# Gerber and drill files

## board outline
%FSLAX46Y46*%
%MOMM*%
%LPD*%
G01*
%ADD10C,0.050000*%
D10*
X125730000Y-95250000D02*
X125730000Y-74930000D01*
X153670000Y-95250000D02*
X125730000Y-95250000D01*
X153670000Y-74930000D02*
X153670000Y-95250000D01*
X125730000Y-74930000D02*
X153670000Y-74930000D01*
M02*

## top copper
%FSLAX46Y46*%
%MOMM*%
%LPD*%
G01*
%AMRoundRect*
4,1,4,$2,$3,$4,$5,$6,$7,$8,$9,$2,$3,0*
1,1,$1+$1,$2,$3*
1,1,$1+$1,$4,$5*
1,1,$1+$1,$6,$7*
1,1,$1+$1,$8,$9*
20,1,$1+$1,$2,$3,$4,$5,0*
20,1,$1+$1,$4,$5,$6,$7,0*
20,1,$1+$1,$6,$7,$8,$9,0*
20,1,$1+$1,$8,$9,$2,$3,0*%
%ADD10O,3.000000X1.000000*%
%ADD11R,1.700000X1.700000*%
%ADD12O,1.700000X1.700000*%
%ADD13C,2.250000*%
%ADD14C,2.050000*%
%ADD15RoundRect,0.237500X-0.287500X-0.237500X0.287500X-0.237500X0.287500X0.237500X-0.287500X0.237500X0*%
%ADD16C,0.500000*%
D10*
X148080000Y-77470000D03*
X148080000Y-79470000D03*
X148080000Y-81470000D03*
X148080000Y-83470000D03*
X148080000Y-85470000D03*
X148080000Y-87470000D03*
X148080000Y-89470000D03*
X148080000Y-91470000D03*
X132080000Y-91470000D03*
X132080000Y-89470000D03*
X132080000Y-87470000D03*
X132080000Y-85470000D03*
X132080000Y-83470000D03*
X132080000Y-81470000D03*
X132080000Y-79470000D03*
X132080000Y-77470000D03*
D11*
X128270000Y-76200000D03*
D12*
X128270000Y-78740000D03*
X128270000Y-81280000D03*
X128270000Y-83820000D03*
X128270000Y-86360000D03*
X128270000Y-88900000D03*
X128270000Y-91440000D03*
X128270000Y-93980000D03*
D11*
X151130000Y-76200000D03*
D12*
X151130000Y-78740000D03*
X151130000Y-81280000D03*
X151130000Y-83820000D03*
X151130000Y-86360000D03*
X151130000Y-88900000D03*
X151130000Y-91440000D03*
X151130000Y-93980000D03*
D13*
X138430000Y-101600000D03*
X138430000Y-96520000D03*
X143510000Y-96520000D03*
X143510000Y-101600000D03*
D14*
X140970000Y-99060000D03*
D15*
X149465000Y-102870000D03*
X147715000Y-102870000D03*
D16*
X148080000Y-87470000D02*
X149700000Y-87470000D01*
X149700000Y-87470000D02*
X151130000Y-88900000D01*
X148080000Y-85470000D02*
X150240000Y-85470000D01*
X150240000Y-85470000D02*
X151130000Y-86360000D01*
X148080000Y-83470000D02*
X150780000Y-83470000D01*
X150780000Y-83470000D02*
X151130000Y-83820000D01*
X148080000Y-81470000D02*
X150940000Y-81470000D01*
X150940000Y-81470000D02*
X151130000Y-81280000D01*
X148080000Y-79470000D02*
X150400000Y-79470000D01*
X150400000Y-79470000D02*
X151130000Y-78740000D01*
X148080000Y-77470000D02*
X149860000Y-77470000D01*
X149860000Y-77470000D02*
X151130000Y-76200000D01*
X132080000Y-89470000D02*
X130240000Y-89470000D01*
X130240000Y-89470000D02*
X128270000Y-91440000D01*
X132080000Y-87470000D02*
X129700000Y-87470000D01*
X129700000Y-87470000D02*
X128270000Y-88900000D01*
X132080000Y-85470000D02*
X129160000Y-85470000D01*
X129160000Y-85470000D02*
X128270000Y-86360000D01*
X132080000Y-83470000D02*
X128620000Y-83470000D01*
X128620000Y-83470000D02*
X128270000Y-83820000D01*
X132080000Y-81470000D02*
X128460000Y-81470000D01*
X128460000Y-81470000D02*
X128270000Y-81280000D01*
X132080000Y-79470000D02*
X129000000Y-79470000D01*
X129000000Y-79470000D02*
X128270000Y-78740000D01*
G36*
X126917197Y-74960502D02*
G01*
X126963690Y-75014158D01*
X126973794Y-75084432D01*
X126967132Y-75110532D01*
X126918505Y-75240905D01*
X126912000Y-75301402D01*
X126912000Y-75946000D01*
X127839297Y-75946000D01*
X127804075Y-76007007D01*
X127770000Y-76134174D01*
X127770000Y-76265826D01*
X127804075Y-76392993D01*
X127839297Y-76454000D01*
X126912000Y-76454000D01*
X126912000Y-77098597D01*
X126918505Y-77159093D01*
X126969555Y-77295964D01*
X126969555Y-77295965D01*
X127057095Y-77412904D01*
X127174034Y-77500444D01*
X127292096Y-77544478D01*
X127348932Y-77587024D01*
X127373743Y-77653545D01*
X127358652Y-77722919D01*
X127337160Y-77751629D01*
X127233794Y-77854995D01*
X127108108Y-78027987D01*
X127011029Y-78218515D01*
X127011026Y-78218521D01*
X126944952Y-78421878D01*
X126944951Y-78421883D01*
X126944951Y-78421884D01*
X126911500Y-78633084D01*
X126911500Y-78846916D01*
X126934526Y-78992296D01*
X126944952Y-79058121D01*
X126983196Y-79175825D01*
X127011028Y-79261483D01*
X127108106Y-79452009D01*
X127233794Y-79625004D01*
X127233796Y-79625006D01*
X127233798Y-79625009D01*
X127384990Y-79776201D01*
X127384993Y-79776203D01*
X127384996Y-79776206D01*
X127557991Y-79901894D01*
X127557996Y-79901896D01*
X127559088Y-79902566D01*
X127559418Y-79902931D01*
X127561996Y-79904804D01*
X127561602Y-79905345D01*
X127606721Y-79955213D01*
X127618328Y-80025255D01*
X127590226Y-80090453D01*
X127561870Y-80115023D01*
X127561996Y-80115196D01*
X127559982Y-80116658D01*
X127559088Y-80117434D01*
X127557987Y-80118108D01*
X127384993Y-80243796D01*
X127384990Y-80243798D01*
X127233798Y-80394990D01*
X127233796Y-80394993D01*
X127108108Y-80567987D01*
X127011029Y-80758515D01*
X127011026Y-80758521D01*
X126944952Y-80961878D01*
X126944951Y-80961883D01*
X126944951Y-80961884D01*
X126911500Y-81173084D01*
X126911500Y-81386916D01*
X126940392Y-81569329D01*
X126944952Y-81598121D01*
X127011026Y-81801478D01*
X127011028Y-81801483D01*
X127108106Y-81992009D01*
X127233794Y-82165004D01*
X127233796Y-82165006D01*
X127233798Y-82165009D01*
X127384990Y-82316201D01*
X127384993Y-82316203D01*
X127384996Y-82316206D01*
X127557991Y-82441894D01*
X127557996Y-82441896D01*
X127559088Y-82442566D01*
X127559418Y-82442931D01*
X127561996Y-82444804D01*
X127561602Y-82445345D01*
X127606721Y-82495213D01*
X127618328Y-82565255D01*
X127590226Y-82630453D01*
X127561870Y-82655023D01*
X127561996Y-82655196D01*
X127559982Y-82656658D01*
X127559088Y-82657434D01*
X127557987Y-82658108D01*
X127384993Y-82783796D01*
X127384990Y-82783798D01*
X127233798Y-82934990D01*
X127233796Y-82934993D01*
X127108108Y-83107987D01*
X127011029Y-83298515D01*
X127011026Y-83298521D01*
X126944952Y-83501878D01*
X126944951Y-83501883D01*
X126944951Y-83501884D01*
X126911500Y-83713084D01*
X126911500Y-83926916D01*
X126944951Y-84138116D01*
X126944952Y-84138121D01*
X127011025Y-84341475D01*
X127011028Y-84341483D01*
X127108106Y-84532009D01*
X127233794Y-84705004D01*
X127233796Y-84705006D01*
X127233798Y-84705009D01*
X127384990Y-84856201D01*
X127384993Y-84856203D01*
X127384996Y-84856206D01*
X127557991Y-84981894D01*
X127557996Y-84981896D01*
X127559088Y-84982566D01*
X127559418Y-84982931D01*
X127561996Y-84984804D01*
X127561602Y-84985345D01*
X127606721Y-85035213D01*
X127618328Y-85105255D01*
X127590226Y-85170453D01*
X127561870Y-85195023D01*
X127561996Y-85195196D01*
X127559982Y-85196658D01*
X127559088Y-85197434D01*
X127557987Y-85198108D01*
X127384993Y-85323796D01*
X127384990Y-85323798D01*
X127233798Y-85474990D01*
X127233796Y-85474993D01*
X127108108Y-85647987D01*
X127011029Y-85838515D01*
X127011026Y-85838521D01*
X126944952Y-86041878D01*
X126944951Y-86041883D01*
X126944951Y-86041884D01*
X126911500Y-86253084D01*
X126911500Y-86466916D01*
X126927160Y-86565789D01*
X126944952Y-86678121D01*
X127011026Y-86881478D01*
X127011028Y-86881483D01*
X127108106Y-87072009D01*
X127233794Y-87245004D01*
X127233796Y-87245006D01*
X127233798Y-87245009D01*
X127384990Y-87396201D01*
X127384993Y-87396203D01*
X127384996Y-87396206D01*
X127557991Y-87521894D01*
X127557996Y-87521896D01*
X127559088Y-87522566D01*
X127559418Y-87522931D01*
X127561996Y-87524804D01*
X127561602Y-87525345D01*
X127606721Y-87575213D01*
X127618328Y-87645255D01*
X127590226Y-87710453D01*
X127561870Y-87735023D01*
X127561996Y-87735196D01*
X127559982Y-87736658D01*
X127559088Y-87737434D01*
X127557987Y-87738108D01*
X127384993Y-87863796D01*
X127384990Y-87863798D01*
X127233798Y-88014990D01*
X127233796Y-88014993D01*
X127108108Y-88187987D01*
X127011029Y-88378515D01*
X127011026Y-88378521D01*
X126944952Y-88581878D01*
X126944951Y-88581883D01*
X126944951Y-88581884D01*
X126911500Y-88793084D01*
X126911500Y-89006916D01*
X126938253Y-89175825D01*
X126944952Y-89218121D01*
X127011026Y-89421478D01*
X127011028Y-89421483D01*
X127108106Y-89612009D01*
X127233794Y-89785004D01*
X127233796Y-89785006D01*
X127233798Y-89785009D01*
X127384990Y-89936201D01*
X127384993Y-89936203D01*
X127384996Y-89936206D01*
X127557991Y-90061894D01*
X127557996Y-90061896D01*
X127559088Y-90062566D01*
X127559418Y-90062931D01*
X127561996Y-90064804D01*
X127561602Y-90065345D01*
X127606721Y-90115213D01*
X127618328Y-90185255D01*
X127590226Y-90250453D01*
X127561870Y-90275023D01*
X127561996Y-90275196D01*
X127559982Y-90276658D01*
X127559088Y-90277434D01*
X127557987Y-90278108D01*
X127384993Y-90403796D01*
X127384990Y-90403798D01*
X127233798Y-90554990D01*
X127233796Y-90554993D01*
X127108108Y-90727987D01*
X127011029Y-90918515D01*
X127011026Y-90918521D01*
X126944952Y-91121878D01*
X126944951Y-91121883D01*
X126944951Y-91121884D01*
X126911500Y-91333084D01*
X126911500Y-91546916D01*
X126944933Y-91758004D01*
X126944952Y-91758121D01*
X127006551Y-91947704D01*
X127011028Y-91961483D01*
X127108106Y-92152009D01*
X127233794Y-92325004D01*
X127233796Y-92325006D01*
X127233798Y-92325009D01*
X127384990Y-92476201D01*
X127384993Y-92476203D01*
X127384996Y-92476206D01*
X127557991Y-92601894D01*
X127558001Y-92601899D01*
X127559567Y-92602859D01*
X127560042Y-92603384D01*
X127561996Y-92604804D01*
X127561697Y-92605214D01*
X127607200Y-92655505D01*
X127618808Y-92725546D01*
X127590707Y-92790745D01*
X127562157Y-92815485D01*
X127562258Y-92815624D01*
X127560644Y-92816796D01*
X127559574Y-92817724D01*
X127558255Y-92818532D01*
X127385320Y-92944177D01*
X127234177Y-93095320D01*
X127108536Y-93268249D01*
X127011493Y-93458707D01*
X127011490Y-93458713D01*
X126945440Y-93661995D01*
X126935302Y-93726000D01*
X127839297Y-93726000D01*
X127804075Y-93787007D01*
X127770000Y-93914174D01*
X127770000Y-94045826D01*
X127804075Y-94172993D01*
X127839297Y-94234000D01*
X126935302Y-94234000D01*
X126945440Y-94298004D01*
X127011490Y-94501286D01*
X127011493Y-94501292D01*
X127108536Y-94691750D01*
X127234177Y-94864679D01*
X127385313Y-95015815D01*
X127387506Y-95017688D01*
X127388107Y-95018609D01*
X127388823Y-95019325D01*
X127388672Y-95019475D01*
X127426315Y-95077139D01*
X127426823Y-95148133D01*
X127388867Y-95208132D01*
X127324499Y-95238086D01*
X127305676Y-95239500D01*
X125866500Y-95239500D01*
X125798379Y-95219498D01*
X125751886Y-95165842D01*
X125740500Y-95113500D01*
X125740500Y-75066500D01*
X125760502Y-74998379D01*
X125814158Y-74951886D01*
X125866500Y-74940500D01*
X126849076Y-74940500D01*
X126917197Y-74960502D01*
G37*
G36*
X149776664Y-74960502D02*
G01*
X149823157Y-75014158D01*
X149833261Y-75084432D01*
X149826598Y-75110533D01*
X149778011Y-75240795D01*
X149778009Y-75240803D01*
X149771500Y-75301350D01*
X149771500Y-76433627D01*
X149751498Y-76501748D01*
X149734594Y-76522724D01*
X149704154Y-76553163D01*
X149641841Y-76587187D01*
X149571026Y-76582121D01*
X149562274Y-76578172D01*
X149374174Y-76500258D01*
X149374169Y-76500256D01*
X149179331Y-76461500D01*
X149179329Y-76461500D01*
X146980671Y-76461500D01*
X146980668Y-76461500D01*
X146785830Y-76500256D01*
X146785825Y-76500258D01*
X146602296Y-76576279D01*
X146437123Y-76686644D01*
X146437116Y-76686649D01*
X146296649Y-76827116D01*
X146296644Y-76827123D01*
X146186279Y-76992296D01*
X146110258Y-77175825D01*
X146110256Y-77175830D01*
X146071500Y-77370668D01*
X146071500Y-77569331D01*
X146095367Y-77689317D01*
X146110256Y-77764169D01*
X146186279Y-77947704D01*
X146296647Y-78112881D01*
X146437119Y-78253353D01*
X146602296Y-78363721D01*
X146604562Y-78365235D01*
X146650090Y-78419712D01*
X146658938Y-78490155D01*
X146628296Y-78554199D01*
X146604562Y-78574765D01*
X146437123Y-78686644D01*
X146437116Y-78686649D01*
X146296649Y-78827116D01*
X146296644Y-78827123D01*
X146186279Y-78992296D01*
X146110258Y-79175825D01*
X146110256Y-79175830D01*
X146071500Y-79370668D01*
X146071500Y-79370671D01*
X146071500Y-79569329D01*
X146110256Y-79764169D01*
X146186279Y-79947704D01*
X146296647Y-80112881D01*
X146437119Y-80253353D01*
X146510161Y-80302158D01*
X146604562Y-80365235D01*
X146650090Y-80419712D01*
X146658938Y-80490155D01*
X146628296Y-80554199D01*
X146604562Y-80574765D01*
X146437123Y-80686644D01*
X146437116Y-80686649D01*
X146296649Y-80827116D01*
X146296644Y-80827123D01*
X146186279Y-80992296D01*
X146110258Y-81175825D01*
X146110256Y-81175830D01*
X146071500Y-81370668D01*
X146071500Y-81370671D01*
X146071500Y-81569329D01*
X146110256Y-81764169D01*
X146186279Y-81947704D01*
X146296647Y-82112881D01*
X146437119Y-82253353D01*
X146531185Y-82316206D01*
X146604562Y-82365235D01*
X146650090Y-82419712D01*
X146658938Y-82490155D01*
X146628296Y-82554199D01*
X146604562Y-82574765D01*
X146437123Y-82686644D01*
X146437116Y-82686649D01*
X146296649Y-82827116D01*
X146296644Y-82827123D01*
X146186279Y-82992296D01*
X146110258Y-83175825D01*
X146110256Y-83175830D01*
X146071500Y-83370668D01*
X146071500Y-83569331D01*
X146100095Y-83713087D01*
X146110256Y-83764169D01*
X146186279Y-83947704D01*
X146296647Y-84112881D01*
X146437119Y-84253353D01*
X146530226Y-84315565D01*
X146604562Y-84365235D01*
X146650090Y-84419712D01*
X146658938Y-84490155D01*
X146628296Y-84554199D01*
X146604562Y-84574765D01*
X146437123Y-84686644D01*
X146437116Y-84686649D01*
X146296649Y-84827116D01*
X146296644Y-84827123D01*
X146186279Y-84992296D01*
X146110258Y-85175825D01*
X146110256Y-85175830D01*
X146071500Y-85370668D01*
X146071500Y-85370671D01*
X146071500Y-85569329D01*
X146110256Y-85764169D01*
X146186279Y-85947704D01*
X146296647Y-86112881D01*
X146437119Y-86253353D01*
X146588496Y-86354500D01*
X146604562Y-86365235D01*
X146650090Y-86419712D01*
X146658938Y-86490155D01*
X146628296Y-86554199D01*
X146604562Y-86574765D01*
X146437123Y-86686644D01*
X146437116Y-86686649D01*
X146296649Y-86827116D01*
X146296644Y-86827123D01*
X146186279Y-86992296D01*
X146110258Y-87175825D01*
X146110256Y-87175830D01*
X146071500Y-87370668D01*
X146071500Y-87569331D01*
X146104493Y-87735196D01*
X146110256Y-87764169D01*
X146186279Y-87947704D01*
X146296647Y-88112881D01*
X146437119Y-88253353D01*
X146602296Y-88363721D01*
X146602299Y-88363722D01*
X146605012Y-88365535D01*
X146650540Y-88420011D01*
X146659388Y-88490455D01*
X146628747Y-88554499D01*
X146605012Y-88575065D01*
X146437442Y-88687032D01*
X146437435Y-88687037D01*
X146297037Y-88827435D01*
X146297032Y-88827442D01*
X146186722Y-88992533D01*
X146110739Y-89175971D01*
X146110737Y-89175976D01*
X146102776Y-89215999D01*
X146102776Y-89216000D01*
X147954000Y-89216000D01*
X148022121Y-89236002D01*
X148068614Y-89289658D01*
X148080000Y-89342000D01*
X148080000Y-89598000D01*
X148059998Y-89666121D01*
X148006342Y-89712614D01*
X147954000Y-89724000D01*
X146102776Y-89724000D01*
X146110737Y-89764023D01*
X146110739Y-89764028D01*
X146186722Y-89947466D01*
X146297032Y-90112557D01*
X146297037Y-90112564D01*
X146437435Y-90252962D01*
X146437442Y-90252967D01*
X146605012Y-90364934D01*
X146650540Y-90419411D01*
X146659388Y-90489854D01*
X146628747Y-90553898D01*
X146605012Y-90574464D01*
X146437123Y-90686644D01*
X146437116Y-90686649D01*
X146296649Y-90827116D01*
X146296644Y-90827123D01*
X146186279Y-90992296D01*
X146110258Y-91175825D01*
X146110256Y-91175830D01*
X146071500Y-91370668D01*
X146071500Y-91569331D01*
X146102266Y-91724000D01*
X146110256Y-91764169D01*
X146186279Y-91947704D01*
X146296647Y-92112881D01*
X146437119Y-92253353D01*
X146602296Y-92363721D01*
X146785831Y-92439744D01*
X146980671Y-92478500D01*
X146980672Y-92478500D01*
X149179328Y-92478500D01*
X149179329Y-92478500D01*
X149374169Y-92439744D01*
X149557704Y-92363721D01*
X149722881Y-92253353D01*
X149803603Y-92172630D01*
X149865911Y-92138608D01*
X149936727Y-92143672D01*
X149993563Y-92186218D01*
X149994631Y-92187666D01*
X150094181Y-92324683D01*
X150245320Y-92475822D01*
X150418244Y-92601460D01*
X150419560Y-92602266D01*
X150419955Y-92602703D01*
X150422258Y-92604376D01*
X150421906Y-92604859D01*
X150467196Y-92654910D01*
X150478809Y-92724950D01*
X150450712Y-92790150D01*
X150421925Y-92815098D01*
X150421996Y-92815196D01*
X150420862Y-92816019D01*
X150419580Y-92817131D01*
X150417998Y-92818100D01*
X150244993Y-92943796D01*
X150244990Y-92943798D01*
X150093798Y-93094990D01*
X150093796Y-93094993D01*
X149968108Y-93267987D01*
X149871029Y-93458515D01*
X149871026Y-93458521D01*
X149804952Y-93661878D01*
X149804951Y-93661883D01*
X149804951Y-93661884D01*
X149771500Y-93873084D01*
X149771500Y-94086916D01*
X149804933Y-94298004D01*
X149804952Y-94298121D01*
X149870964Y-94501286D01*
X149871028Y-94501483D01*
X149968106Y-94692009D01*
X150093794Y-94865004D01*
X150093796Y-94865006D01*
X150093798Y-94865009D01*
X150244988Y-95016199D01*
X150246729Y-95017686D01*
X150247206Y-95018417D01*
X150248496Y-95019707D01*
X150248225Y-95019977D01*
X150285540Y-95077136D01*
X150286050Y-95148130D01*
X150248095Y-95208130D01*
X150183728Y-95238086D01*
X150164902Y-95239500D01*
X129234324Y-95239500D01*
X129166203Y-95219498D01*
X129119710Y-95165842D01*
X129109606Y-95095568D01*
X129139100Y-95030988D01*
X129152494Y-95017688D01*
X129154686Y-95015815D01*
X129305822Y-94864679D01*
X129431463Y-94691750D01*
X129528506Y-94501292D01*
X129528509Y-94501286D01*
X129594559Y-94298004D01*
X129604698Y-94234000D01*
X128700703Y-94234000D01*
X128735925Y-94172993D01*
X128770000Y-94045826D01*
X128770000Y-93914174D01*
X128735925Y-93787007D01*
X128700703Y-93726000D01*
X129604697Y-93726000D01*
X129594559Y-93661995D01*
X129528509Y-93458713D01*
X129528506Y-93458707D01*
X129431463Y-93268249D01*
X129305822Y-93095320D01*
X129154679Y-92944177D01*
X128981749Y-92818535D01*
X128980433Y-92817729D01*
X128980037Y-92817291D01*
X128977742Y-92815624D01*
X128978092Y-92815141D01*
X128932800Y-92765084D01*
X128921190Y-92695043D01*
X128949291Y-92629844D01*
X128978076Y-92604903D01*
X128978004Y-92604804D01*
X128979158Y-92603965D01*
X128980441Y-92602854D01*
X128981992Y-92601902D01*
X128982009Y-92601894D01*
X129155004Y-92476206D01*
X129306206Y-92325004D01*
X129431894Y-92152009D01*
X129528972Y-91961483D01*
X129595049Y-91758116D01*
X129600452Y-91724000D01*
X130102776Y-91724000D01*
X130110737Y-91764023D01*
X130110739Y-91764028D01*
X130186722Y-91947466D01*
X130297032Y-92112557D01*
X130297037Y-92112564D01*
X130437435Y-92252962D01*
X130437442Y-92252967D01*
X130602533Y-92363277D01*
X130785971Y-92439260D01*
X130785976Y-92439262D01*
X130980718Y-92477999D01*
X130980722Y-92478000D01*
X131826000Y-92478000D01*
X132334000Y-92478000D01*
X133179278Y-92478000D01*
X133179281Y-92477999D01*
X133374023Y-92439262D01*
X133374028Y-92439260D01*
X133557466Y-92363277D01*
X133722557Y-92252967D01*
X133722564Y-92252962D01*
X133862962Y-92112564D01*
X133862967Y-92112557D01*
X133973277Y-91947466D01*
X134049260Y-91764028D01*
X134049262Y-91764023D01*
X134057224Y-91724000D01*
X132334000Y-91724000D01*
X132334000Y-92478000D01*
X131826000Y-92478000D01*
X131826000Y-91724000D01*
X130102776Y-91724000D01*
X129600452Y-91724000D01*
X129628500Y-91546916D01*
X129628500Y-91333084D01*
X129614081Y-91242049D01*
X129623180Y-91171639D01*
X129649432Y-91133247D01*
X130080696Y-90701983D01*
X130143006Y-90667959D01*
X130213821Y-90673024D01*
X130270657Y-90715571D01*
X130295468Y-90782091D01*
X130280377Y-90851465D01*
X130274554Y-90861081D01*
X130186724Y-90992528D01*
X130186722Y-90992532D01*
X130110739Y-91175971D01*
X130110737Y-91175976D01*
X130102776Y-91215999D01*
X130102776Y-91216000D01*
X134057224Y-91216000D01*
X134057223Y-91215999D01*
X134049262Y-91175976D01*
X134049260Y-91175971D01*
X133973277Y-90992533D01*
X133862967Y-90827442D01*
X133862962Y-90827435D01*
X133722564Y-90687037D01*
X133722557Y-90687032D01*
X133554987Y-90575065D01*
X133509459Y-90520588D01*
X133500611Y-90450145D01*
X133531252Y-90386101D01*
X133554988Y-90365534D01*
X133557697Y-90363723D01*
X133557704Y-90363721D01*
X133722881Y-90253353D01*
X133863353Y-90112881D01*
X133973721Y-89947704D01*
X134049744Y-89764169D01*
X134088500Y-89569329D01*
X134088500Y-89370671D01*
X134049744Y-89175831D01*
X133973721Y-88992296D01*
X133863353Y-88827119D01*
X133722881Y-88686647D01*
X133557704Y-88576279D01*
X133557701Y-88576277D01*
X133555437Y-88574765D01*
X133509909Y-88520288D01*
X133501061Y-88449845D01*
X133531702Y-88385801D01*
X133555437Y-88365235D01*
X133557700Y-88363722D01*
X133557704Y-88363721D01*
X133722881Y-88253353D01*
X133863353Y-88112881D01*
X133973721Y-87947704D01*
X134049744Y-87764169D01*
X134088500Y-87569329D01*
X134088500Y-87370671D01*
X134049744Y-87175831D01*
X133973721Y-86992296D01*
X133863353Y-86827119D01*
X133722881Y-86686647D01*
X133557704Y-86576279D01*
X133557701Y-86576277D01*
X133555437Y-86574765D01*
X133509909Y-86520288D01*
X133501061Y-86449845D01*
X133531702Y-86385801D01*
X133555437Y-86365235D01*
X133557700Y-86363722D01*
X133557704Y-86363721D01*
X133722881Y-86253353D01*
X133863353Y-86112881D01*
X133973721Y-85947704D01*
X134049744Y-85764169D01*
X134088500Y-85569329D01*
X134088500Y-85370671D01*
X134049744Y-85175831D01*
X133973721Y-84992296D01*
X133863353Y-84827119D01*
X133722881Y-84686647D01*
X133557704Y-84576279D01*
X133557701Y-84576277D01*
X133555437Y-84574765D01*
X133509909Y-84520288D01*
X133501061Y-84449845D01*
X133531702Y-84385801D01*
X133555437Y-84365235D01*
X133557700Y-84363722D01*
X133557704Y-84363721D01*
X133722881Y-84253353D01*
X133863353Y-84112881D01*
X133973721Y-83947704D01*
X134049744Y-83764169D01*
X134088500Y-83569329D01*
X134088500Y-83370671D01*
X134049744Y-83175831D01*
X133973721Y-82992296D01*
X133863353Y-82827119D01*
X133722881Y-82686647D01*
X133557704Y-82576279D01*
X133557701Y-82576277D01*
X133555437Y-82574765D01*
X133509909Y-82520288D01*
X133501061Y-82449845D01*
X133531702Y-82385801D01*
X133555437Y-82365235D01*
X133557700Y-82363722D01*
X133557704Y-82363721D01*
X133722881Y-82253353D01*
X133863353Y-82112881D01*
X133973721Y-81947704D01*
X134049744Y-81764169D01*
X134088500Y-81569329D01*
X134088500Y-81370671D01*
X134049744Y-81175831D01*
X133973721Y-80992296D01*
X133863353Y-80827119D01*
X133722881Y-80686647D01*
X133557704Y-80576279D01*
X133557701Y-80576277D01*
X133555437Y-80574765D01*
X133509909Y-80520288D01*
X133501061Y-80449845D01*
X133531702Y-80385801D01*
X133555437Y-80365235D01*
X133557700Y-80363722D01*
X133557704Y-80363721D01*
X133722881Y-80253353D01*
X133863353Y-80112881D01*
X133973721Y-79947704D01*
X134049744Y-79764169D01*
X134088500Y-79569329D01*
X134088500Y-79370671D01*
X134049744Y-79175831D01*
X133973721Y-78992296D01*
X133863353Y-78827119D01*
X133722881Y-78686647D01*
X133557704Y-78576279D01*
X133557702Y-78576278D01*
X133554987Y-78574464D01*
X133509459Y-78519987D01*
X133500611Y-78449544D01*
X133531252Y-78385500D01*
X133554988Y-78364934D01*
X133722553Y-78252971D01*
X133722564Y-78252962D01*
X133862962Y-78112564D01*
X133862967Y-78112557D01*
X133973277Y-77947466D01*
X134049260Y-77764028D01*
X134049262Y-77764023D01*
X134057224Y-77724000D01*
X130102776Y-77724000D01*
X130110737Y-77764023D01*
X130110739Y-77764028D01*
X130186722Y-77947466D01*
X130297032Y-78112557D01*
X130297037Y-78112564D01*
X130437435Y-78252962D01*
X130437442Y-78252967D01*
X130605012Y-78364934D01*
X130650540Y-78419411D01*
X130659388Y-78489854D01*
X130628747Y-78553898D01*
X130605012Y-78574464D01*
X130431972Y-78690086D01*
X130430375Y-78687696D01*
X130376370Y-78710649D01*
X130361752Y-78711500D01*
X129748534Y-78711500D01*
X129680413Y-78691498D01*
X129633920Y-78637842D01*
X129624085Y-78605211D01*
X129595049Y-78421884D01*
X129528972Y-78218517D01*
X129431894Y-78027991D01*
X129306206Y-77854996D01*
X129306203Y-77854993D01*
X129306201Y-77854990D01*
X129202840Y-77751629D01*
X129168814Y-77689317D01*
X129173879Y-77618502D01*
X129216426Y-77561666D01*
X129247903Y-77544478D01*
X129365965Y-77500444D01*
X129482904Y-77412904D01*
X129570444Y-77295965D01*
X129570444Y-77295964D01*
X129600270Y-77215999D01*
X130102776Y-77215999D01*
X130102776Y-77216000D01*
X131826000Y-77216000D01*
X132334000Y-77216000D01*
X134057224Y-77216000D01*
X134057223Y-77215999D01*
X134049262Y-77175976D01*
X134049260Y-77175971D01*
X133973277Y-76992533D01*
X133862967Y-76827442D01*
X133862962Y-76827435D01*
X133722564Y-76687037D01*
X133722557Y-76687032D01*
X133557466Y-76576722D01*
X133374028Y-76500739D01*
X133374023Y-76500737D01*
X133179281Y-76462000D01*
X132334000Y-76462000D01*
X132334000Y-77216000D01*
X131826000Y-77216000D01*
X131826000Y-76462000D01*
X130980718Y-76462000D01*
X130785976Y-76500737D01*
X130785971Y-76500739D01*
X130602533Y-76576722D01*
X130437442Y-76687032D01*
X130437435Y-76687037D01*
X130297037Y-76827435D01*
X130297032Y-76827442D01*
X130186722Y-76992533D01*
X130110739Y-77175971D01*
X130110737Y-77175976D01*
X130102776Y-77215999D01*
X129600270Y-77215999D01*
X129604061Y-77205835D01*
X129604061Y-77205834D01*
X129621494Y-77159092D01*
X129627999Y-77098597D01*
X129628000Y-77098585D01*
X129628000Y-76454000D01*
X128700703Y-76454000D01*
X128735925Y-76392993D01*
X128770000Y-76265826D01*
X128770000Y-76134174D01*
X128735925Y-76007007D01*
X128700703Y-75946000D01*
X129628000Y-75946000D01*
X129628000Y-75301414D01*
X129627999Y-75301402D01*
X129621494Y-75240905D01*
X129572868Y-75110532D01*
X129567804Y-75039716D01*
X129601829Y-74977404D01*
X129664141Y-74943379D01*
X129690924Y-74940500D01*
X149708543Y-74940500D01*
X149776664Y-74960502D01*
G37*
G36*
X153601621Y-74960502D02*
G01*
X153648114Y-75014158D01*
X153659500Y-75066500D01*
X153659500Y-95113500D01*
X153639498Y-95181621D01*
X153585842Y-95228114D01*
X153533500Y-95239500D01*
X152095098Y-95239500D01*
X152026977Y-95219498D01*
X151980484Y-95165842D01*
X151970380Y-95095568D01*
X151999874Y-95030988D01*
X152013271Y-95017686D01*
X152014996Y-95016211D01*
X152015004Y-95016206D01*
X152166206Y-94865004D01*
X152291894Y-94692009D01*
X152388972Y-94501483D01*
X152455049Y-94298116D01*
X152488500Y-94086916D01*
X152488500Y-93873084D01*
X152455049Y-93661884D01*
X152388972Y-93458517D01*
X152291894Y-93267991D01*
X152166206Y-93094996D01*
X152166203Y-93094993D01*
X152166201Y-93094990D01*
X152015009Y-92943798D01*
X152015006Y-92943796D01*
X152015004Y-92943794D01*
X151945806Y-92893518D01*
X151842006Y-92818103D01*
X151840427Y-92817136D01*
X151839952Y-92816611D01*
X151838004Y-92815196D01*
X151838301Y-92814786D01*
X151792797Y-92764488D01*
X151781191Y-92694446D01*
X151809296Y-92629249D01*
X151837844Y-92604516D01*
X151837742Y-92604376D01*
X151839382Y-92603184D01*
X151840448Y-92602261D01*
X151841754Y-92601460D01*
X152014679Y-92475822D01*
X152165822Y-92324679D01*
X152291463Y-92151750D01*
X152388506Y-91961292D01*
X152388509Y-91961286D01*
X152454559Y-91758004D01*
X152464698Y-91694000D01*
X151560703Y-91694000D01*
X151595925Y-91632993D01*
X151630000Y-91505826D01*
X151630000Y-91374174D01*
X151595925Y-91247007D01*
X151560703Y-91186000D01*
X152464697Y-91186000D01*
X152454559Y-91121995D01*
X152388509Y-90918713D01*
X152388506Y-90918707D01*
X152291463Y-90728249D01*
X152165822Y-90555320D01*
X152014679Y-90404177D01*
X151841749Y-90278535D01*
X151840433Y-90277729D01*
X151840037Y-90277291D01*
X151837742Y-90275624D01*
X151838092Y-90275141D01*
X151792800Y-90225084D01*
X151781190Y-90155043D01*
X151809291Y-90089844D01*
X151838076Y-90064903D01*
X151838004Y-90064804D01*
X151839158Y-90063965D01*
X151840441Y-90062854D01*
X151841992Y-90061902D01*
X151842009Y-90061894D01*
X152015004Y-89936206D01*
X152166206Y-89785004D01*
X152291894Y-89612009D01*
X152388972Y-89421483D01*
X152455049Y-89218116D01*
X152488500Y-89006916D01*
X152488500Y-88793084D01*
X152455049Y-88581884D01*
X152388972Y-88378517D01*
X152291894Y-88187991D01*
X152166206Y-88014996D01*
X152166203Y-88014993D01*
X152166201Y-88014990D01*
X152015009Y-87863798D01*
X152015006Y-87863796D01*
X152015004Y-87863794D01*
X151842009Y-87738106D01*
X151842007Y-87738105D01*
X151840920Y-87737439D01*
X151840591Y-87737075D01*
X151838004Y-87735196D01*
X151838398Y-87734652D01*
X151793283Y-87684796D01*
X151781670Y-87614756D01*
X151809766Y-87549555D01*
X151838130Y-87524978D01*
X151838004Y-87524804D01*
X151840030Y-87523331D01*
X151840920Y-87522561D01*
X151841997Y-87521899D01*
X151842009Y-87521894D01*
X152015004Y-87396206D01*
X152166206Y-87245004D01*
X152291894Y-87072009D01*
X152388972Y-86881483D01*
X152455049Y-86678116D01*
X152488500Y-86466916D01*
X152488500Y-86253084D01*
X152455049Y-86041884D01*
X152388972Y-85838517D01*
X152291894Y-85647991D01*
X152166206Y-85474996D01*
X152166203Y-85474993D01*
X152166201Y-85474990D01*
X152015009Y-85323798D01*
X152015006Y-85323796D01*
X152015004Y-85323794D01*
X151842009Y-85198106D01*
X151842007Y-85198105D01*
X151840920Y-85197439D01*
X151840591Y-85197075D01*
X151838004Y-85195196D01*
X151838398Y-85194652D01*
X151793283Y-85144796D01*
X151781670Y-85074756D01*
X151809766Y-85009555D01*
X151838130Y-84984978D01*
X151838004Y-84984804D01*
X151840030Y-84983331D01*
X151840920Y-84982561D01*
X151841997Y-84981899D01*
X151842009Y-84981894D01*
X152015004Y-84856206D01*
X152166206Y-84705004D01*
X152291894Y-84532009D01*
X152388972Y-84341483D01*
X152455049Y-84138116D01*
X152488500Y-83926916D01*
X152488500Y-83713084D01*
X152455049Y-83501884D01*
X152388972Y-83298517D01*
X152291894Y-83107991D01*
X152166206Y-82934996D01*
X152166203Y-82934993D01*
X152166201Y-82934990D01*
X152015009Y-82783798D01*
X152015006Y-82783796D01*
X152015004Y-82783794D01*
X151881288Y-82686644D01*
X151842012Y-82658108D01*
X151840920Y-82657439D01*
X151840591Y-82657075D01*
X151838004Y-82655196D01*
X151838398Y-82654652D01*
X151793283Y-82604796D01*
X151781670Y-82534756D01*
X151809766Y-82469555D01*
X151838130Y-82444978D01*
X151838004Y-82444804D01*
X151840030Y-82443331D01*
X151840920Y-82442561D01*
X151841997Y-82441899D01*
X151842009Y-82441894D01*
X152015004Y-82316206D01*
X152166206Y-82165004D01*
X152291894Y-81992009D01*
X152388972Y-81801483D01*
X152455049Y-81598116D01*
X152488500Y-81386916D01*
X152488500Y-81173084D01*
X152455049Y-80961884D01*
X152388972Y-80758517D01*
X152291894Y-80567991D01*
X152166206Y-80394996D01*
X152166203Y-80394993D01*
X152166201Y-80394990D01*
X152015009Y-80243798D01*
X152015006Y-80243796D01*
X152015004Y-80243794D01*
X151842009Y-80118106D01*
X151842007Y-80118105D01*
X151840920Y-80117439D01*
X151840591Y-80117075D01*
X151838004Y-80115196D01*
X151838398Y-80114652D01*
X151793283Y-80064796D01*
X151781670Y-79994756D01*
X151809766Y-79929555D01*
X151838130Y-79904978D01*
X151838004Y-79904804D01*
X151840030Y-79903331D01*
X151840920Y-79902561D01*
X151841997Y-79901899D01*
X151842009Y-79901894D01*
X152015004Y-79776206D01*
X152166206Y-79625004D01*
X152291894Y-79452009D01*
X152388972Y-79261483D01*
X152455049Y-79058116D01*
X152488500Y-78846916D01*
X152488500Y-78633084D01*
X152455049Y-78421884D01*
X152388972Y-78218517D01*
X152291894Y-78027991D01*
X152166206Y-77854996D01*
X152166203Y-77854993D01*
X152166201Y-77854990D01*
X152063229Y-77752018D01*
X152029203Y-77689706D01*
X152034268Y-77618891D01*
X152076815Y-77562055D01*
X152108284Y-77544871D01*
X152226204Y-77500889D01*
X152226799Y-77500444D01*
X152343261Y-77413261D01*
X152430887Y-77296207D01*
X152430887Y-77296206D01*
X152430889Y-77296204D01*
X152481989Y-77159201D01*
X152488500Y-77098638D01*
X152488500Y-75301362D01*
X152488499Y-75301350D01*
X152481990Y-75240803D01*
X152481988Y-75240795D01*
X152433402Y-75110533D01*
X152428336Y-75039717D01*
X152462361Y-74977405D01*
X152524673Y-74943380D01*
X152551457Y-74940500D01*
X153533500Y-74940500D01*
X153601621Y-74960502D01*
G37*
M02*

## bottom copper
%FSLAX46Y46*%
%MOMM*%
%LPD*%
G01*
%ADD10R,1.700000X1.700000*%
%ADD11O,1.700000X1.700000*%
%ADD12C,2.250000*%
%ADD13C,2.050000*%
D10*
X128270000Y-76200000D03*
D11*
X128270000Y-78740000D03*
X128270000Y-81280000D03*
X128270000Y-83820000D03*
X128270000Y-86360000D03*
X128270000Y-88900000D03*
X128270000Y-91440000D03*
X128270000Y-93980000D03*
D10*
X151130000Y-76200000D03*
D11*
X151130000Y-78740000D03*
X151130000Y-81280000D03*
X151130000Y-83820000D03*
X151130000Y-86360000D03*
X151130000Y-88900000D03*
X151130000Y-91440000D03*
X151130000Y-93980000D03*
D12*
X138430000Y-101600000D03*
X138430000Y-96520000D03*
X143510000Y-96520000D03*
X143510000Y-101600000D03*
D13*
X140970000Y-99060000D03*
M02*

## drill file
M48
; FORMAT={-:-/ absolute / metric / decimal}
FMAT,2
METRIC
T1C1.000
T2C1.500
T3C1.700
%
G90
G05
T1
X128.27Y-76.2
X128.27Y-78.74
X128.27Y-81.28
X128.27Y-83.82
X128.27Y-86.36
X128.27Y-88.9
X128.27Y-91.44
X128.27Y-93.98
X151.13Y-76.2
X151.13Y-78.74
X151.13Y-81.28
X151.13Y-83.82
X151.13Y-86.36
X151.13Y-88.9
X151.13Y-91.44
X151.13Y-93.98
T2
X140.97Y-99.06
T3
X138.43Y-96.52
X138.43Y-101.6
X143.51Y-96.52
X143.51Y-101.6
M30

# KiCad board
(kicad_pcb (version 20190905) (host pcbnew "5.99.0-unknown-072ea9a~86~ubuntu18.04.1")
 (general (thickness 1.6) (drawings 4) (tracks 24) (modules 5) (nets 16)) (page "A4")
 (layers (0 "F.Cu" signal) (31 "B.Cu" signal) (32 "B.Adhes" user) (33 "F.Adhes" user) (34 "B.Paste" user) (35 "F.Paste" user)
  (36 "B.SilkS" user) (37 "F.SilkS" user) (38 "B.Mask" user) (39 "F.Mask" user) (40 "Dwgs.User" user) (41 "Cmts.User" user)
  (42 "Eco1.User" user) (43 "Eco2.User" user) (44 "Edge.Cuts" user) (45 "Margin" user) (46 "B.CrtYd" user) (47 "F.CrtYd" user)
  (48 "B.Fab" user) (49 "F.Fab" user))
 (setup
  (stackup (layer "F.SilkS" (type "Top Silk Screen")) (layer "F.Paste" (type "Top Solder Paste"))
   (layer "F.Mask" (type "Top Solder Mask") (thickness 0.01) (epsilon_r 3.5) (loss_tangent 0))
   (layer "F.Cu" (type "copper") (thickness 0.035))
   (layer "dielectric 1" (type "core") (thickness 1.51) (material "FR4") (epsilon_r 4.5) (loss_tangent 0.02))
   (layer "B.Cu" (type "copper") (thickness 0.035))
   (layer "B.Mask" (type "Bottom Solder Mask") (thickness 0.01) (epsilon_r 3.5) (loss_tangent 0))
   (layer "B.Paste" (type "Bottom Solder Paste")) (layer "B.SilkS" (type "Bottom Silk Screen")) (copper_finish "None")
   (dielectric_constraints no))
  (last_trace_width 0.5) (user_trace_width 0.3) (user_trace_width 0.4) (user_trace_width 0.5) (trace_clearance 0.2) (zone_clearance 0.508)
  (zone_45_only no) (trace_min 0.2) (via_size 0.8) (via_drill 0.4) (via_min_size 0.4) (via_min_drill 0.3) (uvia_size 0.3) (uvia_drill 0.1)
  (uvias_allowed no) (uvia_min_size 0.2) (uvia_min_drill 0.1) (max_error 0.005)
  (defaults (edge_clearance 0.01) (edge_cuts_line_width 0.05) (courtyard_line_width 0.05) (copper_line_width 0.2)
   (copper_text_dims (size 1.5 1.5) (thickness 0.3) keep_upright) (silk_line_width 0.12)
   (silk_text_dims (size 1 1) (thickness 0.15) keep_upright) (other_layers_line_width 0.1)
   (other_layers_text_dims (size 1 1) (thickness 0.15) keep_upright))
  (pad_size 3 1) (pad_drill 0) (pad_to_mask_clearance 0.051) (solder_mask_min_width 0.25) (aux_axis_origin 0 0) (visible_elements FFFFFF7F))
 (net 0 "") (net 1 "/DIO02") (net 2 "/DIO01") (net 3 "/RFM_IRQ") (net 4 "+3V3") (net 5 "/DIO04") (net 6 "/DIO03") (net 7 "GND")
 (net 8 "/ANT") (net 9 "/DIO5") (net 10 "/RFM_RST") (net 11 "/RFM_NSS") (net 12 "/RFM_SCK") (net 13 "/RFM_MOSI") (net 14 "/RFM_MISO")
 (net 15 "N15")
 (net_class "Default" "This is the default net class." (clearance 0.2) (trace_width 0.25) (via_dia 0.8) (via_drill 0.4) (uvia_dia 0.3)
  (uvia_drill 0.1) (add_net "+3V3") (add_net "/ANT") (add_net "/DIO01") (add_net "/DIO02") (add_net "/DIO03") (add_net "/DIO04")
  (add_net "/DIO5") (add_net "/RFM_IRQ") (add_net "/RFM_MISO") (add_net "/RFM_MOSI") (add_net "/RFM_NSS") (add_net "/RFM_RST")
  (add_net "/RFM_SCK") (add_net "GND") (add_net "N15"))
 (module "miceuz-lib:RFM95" (layer "F.Cu") (at 132.08 77.47)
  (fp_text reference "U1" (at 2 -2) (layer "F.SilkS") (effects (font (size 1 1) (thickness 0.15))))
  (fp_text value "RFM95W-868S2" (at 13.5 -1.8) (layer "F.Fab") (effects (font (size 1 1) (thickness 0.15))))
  (pad "16" smd oval (at 16 0) (size 3 1) (layers "F.Cu" "F.Paste" "F.Mask") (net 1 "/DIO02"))
  (pad "15" smd oval (at 16 2) (size 3 1) (layers "F.Cu" "F.Paste" "F.Mask") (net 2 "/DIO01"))
  (pad "14" smd oval (at 16 4) (size 3 1) (layers "F.Cu" "F.Paste" "F.Mask") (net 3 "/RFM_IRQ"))
  (pad "13" smd oval (at 16 6) (size 3 1) (layers "F.Cu" "F.Paste" "F.Mask") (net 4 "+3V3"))
  (pad "12" smd oval (at 16 8) (size 3 1) (layers "F.Cu" "F.Paste" "F.Mask") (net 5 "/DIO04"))
  (pad "11" smd oval (at 16 10) (size 3 1) (layers "F.Cu" "F.Paste" "F.Mask") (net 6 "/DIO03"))
  (pad "10" smd oval (at 16 12) (size 3 1) (layers "F.Cu" "F.Paste" "F.Mask") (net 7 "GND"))
  (pad "9" smd oval (at 16 14) (size 3 1) (layers "F.Cu" "F.Paste" "F.Mask") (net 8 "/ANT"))
  (pad "8" smd oval (at 0 14) (size 3 1) (layers "F.Cu" "F.Paste" "F.Mask") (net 7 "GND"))
  (pad "7" smd oval (at 0 12) (size 3 1) (layers "F.Cu" "F.Paste" "F.Mask") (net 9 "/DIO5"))
  (pad "6" smd oval (at 0 10) (size 3 1) (layers "F.Cu" "F.Paste" "F.Mask") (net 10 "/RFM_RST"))
  (pad "5" smd oval (at 0 8) (size 3 1) (layers "F.Cu" "F.Paste" "F.Mask") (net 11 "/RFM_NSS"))
  (pad "4" smd oval (at 0 6) (size 3 1) (layers "F.Cu" "F.Paste" "F.Mask") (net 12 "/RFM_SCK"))
  (pad "3" smd oval (at 0 4) (size 3 1) (layers "F.Cu" "F.Paste" "F.Mask") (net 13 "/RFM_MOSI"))
  (pad "2" smd oval (at 0 2) (size 3 1) (layers "F.Cu" "F.Paste" "F.Mask") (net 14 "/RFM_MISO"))
  (pad "1" smd oval (at 0 0) (size 3 1) (layers "F.Cu" "F.Paste" "F.Mask") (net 7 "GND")))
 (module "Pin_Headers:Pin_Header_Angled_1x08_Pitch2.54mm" (layer "F.Cu") (at 128.27 76.2)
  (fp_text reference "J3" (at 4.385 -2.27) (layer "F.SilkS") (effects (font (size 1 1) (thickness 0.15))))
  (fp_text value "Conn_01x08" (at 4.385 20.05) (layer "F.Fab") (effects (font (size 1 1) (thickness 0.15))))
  (pad "1" thru_hole rect (at 0 0) (size 1.7 1.7) (drill 1) (layers *.Cu *.Mask) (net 7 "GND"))
  (pad "2" thru_hole oval (at 0 2.54) (size 1.7 1.7) (drill 1) (layers *.Cu *.Mask) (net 14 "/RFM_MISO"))
  (pad "3" thru_hole oval (at 0 5.08) (size 1.7 1.7) (drill 1) (layers *.Cu *.Mask) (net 13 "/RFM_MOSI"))
  (pad "4" thru_hole oval (at 0 7.62) (size 1.7 1.7) (drill 1) (layers *.Cu *.Mask) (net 12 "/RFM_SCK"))
  (pad "5" thru_hole oval (at 0 10.16) (size 1.7 1.7) (drill 1) (layers *.Cu *.Mask) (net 11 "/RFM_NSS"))
  (pad "6" thru_hole oval (at 0 12.7) (size 1.7 1.7) (drill 1) (layers *.Cu *.Mask) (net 10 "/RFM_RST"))
  (pad "7" thru_hole oval (at 0 15.24) (size 1.7 1.7) (drill 1) (layers *.Cu *.Mask) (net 9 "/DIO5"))
  (pad "8" thru_hole oval (at 0 17.78) (size 1.7 1.7) (drill 1) (layers *.Cu *.Mask) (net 7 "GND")))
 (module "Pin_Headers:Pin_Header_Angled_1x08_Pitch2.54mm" (layer "F.Cu") (at 151.13 76.2)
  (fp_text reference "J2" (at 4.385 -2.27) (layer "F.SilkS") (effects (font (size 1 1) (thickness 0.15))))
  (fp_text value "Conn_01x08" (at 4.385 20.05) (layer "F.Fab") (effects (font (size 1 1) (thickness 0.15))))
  (pad "1" thru_hole rect (at 0 0) (size 1.7 1.7) (drill 1) (layers *.Cu *.Mask) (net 1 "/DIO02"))
  (pad "2" thru_hole oval (at 0 2.54) (size 1.7 1.7) (drill 1) (layers *.Cu *.Mask) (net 2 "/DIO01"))
  (pad "3" thru_hole oval (at 0 5.08) (size 1.7 1.7) (drill 1) (layers *.Cu *.Mask) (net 3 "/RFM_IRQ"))
  (pad "4" thru_hole oval (at 0 7.62) (size 1.7 1.7) (drill 1) (layers *.Cu *.Mask) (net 4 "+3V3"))
  (pad "5" thru_hole oval (at 0 10.16) (size 1.7 1.7) (drill 1) (layers *.Cu *.Mask) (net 5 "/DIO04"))
  (pad "6" thru_hole oval (at 0 12.7) (size 1.7 1.7) (drill 1) (layers *.Cu *.Mask) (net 6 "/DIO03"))
  (pad "7" thru_hole oval (at 0 15.24) (size 1.7 1.7) (drill 1) (layers *.Cu *.Mask) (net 7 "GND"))
  (pad "8" thru_hole oval (at 0 17.78) (size 1.7 1.7) (drill 1) (layers *.Cu *.Mask) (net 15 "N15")))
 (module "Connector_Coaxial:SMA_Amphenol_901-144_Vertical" (layer "F.Cu") (at 140.97 99.06)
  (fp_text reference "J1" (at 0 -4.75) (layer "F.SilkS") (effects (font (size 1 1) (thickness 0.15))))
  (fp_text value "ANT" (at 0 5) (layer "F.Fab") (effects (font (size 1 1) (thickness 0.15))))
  (pad "2" thru_hole circle (at -2.54 2.54) (size 2.25 2.25) (drill 1.7) (layers *.Cu *.Mask) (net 7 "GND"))
  (pad "2" thru_hole circle (at -2.54 -2.54) (size 2.25 2.25) (drill 1.7) (layers *.Cu *.Mask) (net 7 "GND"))
  (pad "2" thru_hole circle (at 2.54 -2.54) (size 2.25 2.25) (drill 1.7) (layers *.Cu *.Mask) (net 7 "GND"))
  (pad "2" thru_hole circle (at 2.54 2.54) (size 2.25 2.25) (drill 1.7) (layers *.Cu *.Mask) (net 7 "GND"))
  (pad "1" thru_hole circle (at 0 0) (size 2.05 2.05) (drill 1.5) (layers *.Cu *.Mask) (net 8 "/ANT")))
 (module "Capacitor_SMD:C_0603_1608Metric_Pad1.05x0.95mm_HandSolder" (layer "F.Cu") (at 148.59 102.87)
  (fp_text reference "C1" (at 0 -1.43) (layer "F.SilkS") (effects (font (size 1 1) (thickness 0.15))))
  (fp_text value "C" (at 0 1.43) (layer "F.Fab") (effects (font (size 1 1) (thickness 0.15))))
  (pad "2" smd roundrect (at 0.875 0) (size 1.05 0.95) (layers "F.Cu" "F.Paste" "F.Mask") (roundrect_rratio 0.25) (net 7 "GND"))
  (pad "1" smd roundrect (at -0.875 0) (size 1.05 0.95) (layers "F.Cu" "F.Paste" "F.Mask") (roundrect_rratio 0.25) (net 4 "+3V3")))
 (gr_line (start 125.73 95.25) (end 125.73 74.93) (layer "Edge.Cuts") (width 0.05))
 (gr_line (start 153.67 95.25) (end 125.73 95.25) (layer "Edge.Cuts") (width 0.05))
 (gr_line (start 153.67 74.93) (end 153.67 95.25) (layer "Edge.Cuts") (width 0.05))
 (gr_line (start 125.73 74.93) (end 153.67 74.93) (layer "Edge.Cuts") (width 0.05))
 (segment (start 148.08 87.47) (end 149.7 87.47) (width 0.5) (layer "F.Cu") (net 6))
 (segment (start 149.7 87.47) (end 151.13 88.9) (width 0.5) (layer "F.Cu") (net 6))
 (segment (start 148.08 85.47) (end 150.24 85.47) (width 0.5) (layer "F.Cu") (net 5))
 (segment (start 150.24 85.47) (end 151.13 86.36) (width 0.5) (layer "F.Cu") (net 5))
 (segment (start 148.08 83.47) (end 150.78 83.47) (width 0.5) (layer "F.Cu") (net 4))
 (segment (start 150.78 83.47) (end 151.13 83.82) (width 0.5) (layer "F.Cu") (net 4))
 (segment (start 148.08 81.47) (end 150.94 81.47) (width 0.5) (layer "F.Cu") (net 3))
 (segment (start 150.94 81.47) (end 151.13 81.28) (width 0.5) (layer "F.Cu") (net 3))
 (segment (start 148.08 79.47) (end 150.4 79.47) (width 0.5) (layer "F.Cu") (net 2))
 (segment (start 150.4 79.47) (end 151.13 78.74) (width 0.5) (layer "F.Cu") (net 2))
 (segment (start 148.08 77.47) (end 149.86 77.47) (width 0.5) (layer "F.Cu") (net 1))
 (segment (start 149.86 77.47) (end 151.13 76.2) (width 0.5) (layer "F.Cu") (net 1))
 (segment (start 132.08 89.47) (end 130.24 89.47) (width 0.5) (layer "F.Cu") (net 9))
 (segment (start 130.24 89.47) (end 128.27 91.44) (width 0.5) (layer "F.Cu") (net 9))
 (segment (start 132.08 87.47) (end 129.7 87.47) (width 0.5) (layer "F.Cu") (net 10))
 (segment (start 129.7 87.47) (end 128.27 88.9) (width 0.5) (layer "F.Cu") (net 10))
 (segment (start 132.08 85.47) (end 129.16 85.47) (width 0.5) (layer "F.Cu") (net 11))
 (segment (start 129.16 85.47) (end 128.27 86.36) (width 0.5) (layer "F.Cu") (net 11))
 (segment (start 132.08 83.47) (end 128.62 83.47) (width 0.5) (layer "F.Cu") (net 12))
 (segment (start 128.62 83.47) (end 128.27 83.82) (width 0.5) (layer "F.Cu") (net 12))
 (segment (start 132.08 81.47) (end 128.46 81.47) (width 0.5) (layer "F.Cu") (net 13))
 (segment (start 128.46 81.47) (end 128.27 81.28) (width 0.5) (layer "F.Cu") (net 13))
 (segment (start 132.08 79.47) (end 129 79.47) (width 0.5) (layer "F.Cu") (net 14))
 (segment (start 129 79.47) (end 128.27 78.74) (width 0.5) (layer "F.Cu") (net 14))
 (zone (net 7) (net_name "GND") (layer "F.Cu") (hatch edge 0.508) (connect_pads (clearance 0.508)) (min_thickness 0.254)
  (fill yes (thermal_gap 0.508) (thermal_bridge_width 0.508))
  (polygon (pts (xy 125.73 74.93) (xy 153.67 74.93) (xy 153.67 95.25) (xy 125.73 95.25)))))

